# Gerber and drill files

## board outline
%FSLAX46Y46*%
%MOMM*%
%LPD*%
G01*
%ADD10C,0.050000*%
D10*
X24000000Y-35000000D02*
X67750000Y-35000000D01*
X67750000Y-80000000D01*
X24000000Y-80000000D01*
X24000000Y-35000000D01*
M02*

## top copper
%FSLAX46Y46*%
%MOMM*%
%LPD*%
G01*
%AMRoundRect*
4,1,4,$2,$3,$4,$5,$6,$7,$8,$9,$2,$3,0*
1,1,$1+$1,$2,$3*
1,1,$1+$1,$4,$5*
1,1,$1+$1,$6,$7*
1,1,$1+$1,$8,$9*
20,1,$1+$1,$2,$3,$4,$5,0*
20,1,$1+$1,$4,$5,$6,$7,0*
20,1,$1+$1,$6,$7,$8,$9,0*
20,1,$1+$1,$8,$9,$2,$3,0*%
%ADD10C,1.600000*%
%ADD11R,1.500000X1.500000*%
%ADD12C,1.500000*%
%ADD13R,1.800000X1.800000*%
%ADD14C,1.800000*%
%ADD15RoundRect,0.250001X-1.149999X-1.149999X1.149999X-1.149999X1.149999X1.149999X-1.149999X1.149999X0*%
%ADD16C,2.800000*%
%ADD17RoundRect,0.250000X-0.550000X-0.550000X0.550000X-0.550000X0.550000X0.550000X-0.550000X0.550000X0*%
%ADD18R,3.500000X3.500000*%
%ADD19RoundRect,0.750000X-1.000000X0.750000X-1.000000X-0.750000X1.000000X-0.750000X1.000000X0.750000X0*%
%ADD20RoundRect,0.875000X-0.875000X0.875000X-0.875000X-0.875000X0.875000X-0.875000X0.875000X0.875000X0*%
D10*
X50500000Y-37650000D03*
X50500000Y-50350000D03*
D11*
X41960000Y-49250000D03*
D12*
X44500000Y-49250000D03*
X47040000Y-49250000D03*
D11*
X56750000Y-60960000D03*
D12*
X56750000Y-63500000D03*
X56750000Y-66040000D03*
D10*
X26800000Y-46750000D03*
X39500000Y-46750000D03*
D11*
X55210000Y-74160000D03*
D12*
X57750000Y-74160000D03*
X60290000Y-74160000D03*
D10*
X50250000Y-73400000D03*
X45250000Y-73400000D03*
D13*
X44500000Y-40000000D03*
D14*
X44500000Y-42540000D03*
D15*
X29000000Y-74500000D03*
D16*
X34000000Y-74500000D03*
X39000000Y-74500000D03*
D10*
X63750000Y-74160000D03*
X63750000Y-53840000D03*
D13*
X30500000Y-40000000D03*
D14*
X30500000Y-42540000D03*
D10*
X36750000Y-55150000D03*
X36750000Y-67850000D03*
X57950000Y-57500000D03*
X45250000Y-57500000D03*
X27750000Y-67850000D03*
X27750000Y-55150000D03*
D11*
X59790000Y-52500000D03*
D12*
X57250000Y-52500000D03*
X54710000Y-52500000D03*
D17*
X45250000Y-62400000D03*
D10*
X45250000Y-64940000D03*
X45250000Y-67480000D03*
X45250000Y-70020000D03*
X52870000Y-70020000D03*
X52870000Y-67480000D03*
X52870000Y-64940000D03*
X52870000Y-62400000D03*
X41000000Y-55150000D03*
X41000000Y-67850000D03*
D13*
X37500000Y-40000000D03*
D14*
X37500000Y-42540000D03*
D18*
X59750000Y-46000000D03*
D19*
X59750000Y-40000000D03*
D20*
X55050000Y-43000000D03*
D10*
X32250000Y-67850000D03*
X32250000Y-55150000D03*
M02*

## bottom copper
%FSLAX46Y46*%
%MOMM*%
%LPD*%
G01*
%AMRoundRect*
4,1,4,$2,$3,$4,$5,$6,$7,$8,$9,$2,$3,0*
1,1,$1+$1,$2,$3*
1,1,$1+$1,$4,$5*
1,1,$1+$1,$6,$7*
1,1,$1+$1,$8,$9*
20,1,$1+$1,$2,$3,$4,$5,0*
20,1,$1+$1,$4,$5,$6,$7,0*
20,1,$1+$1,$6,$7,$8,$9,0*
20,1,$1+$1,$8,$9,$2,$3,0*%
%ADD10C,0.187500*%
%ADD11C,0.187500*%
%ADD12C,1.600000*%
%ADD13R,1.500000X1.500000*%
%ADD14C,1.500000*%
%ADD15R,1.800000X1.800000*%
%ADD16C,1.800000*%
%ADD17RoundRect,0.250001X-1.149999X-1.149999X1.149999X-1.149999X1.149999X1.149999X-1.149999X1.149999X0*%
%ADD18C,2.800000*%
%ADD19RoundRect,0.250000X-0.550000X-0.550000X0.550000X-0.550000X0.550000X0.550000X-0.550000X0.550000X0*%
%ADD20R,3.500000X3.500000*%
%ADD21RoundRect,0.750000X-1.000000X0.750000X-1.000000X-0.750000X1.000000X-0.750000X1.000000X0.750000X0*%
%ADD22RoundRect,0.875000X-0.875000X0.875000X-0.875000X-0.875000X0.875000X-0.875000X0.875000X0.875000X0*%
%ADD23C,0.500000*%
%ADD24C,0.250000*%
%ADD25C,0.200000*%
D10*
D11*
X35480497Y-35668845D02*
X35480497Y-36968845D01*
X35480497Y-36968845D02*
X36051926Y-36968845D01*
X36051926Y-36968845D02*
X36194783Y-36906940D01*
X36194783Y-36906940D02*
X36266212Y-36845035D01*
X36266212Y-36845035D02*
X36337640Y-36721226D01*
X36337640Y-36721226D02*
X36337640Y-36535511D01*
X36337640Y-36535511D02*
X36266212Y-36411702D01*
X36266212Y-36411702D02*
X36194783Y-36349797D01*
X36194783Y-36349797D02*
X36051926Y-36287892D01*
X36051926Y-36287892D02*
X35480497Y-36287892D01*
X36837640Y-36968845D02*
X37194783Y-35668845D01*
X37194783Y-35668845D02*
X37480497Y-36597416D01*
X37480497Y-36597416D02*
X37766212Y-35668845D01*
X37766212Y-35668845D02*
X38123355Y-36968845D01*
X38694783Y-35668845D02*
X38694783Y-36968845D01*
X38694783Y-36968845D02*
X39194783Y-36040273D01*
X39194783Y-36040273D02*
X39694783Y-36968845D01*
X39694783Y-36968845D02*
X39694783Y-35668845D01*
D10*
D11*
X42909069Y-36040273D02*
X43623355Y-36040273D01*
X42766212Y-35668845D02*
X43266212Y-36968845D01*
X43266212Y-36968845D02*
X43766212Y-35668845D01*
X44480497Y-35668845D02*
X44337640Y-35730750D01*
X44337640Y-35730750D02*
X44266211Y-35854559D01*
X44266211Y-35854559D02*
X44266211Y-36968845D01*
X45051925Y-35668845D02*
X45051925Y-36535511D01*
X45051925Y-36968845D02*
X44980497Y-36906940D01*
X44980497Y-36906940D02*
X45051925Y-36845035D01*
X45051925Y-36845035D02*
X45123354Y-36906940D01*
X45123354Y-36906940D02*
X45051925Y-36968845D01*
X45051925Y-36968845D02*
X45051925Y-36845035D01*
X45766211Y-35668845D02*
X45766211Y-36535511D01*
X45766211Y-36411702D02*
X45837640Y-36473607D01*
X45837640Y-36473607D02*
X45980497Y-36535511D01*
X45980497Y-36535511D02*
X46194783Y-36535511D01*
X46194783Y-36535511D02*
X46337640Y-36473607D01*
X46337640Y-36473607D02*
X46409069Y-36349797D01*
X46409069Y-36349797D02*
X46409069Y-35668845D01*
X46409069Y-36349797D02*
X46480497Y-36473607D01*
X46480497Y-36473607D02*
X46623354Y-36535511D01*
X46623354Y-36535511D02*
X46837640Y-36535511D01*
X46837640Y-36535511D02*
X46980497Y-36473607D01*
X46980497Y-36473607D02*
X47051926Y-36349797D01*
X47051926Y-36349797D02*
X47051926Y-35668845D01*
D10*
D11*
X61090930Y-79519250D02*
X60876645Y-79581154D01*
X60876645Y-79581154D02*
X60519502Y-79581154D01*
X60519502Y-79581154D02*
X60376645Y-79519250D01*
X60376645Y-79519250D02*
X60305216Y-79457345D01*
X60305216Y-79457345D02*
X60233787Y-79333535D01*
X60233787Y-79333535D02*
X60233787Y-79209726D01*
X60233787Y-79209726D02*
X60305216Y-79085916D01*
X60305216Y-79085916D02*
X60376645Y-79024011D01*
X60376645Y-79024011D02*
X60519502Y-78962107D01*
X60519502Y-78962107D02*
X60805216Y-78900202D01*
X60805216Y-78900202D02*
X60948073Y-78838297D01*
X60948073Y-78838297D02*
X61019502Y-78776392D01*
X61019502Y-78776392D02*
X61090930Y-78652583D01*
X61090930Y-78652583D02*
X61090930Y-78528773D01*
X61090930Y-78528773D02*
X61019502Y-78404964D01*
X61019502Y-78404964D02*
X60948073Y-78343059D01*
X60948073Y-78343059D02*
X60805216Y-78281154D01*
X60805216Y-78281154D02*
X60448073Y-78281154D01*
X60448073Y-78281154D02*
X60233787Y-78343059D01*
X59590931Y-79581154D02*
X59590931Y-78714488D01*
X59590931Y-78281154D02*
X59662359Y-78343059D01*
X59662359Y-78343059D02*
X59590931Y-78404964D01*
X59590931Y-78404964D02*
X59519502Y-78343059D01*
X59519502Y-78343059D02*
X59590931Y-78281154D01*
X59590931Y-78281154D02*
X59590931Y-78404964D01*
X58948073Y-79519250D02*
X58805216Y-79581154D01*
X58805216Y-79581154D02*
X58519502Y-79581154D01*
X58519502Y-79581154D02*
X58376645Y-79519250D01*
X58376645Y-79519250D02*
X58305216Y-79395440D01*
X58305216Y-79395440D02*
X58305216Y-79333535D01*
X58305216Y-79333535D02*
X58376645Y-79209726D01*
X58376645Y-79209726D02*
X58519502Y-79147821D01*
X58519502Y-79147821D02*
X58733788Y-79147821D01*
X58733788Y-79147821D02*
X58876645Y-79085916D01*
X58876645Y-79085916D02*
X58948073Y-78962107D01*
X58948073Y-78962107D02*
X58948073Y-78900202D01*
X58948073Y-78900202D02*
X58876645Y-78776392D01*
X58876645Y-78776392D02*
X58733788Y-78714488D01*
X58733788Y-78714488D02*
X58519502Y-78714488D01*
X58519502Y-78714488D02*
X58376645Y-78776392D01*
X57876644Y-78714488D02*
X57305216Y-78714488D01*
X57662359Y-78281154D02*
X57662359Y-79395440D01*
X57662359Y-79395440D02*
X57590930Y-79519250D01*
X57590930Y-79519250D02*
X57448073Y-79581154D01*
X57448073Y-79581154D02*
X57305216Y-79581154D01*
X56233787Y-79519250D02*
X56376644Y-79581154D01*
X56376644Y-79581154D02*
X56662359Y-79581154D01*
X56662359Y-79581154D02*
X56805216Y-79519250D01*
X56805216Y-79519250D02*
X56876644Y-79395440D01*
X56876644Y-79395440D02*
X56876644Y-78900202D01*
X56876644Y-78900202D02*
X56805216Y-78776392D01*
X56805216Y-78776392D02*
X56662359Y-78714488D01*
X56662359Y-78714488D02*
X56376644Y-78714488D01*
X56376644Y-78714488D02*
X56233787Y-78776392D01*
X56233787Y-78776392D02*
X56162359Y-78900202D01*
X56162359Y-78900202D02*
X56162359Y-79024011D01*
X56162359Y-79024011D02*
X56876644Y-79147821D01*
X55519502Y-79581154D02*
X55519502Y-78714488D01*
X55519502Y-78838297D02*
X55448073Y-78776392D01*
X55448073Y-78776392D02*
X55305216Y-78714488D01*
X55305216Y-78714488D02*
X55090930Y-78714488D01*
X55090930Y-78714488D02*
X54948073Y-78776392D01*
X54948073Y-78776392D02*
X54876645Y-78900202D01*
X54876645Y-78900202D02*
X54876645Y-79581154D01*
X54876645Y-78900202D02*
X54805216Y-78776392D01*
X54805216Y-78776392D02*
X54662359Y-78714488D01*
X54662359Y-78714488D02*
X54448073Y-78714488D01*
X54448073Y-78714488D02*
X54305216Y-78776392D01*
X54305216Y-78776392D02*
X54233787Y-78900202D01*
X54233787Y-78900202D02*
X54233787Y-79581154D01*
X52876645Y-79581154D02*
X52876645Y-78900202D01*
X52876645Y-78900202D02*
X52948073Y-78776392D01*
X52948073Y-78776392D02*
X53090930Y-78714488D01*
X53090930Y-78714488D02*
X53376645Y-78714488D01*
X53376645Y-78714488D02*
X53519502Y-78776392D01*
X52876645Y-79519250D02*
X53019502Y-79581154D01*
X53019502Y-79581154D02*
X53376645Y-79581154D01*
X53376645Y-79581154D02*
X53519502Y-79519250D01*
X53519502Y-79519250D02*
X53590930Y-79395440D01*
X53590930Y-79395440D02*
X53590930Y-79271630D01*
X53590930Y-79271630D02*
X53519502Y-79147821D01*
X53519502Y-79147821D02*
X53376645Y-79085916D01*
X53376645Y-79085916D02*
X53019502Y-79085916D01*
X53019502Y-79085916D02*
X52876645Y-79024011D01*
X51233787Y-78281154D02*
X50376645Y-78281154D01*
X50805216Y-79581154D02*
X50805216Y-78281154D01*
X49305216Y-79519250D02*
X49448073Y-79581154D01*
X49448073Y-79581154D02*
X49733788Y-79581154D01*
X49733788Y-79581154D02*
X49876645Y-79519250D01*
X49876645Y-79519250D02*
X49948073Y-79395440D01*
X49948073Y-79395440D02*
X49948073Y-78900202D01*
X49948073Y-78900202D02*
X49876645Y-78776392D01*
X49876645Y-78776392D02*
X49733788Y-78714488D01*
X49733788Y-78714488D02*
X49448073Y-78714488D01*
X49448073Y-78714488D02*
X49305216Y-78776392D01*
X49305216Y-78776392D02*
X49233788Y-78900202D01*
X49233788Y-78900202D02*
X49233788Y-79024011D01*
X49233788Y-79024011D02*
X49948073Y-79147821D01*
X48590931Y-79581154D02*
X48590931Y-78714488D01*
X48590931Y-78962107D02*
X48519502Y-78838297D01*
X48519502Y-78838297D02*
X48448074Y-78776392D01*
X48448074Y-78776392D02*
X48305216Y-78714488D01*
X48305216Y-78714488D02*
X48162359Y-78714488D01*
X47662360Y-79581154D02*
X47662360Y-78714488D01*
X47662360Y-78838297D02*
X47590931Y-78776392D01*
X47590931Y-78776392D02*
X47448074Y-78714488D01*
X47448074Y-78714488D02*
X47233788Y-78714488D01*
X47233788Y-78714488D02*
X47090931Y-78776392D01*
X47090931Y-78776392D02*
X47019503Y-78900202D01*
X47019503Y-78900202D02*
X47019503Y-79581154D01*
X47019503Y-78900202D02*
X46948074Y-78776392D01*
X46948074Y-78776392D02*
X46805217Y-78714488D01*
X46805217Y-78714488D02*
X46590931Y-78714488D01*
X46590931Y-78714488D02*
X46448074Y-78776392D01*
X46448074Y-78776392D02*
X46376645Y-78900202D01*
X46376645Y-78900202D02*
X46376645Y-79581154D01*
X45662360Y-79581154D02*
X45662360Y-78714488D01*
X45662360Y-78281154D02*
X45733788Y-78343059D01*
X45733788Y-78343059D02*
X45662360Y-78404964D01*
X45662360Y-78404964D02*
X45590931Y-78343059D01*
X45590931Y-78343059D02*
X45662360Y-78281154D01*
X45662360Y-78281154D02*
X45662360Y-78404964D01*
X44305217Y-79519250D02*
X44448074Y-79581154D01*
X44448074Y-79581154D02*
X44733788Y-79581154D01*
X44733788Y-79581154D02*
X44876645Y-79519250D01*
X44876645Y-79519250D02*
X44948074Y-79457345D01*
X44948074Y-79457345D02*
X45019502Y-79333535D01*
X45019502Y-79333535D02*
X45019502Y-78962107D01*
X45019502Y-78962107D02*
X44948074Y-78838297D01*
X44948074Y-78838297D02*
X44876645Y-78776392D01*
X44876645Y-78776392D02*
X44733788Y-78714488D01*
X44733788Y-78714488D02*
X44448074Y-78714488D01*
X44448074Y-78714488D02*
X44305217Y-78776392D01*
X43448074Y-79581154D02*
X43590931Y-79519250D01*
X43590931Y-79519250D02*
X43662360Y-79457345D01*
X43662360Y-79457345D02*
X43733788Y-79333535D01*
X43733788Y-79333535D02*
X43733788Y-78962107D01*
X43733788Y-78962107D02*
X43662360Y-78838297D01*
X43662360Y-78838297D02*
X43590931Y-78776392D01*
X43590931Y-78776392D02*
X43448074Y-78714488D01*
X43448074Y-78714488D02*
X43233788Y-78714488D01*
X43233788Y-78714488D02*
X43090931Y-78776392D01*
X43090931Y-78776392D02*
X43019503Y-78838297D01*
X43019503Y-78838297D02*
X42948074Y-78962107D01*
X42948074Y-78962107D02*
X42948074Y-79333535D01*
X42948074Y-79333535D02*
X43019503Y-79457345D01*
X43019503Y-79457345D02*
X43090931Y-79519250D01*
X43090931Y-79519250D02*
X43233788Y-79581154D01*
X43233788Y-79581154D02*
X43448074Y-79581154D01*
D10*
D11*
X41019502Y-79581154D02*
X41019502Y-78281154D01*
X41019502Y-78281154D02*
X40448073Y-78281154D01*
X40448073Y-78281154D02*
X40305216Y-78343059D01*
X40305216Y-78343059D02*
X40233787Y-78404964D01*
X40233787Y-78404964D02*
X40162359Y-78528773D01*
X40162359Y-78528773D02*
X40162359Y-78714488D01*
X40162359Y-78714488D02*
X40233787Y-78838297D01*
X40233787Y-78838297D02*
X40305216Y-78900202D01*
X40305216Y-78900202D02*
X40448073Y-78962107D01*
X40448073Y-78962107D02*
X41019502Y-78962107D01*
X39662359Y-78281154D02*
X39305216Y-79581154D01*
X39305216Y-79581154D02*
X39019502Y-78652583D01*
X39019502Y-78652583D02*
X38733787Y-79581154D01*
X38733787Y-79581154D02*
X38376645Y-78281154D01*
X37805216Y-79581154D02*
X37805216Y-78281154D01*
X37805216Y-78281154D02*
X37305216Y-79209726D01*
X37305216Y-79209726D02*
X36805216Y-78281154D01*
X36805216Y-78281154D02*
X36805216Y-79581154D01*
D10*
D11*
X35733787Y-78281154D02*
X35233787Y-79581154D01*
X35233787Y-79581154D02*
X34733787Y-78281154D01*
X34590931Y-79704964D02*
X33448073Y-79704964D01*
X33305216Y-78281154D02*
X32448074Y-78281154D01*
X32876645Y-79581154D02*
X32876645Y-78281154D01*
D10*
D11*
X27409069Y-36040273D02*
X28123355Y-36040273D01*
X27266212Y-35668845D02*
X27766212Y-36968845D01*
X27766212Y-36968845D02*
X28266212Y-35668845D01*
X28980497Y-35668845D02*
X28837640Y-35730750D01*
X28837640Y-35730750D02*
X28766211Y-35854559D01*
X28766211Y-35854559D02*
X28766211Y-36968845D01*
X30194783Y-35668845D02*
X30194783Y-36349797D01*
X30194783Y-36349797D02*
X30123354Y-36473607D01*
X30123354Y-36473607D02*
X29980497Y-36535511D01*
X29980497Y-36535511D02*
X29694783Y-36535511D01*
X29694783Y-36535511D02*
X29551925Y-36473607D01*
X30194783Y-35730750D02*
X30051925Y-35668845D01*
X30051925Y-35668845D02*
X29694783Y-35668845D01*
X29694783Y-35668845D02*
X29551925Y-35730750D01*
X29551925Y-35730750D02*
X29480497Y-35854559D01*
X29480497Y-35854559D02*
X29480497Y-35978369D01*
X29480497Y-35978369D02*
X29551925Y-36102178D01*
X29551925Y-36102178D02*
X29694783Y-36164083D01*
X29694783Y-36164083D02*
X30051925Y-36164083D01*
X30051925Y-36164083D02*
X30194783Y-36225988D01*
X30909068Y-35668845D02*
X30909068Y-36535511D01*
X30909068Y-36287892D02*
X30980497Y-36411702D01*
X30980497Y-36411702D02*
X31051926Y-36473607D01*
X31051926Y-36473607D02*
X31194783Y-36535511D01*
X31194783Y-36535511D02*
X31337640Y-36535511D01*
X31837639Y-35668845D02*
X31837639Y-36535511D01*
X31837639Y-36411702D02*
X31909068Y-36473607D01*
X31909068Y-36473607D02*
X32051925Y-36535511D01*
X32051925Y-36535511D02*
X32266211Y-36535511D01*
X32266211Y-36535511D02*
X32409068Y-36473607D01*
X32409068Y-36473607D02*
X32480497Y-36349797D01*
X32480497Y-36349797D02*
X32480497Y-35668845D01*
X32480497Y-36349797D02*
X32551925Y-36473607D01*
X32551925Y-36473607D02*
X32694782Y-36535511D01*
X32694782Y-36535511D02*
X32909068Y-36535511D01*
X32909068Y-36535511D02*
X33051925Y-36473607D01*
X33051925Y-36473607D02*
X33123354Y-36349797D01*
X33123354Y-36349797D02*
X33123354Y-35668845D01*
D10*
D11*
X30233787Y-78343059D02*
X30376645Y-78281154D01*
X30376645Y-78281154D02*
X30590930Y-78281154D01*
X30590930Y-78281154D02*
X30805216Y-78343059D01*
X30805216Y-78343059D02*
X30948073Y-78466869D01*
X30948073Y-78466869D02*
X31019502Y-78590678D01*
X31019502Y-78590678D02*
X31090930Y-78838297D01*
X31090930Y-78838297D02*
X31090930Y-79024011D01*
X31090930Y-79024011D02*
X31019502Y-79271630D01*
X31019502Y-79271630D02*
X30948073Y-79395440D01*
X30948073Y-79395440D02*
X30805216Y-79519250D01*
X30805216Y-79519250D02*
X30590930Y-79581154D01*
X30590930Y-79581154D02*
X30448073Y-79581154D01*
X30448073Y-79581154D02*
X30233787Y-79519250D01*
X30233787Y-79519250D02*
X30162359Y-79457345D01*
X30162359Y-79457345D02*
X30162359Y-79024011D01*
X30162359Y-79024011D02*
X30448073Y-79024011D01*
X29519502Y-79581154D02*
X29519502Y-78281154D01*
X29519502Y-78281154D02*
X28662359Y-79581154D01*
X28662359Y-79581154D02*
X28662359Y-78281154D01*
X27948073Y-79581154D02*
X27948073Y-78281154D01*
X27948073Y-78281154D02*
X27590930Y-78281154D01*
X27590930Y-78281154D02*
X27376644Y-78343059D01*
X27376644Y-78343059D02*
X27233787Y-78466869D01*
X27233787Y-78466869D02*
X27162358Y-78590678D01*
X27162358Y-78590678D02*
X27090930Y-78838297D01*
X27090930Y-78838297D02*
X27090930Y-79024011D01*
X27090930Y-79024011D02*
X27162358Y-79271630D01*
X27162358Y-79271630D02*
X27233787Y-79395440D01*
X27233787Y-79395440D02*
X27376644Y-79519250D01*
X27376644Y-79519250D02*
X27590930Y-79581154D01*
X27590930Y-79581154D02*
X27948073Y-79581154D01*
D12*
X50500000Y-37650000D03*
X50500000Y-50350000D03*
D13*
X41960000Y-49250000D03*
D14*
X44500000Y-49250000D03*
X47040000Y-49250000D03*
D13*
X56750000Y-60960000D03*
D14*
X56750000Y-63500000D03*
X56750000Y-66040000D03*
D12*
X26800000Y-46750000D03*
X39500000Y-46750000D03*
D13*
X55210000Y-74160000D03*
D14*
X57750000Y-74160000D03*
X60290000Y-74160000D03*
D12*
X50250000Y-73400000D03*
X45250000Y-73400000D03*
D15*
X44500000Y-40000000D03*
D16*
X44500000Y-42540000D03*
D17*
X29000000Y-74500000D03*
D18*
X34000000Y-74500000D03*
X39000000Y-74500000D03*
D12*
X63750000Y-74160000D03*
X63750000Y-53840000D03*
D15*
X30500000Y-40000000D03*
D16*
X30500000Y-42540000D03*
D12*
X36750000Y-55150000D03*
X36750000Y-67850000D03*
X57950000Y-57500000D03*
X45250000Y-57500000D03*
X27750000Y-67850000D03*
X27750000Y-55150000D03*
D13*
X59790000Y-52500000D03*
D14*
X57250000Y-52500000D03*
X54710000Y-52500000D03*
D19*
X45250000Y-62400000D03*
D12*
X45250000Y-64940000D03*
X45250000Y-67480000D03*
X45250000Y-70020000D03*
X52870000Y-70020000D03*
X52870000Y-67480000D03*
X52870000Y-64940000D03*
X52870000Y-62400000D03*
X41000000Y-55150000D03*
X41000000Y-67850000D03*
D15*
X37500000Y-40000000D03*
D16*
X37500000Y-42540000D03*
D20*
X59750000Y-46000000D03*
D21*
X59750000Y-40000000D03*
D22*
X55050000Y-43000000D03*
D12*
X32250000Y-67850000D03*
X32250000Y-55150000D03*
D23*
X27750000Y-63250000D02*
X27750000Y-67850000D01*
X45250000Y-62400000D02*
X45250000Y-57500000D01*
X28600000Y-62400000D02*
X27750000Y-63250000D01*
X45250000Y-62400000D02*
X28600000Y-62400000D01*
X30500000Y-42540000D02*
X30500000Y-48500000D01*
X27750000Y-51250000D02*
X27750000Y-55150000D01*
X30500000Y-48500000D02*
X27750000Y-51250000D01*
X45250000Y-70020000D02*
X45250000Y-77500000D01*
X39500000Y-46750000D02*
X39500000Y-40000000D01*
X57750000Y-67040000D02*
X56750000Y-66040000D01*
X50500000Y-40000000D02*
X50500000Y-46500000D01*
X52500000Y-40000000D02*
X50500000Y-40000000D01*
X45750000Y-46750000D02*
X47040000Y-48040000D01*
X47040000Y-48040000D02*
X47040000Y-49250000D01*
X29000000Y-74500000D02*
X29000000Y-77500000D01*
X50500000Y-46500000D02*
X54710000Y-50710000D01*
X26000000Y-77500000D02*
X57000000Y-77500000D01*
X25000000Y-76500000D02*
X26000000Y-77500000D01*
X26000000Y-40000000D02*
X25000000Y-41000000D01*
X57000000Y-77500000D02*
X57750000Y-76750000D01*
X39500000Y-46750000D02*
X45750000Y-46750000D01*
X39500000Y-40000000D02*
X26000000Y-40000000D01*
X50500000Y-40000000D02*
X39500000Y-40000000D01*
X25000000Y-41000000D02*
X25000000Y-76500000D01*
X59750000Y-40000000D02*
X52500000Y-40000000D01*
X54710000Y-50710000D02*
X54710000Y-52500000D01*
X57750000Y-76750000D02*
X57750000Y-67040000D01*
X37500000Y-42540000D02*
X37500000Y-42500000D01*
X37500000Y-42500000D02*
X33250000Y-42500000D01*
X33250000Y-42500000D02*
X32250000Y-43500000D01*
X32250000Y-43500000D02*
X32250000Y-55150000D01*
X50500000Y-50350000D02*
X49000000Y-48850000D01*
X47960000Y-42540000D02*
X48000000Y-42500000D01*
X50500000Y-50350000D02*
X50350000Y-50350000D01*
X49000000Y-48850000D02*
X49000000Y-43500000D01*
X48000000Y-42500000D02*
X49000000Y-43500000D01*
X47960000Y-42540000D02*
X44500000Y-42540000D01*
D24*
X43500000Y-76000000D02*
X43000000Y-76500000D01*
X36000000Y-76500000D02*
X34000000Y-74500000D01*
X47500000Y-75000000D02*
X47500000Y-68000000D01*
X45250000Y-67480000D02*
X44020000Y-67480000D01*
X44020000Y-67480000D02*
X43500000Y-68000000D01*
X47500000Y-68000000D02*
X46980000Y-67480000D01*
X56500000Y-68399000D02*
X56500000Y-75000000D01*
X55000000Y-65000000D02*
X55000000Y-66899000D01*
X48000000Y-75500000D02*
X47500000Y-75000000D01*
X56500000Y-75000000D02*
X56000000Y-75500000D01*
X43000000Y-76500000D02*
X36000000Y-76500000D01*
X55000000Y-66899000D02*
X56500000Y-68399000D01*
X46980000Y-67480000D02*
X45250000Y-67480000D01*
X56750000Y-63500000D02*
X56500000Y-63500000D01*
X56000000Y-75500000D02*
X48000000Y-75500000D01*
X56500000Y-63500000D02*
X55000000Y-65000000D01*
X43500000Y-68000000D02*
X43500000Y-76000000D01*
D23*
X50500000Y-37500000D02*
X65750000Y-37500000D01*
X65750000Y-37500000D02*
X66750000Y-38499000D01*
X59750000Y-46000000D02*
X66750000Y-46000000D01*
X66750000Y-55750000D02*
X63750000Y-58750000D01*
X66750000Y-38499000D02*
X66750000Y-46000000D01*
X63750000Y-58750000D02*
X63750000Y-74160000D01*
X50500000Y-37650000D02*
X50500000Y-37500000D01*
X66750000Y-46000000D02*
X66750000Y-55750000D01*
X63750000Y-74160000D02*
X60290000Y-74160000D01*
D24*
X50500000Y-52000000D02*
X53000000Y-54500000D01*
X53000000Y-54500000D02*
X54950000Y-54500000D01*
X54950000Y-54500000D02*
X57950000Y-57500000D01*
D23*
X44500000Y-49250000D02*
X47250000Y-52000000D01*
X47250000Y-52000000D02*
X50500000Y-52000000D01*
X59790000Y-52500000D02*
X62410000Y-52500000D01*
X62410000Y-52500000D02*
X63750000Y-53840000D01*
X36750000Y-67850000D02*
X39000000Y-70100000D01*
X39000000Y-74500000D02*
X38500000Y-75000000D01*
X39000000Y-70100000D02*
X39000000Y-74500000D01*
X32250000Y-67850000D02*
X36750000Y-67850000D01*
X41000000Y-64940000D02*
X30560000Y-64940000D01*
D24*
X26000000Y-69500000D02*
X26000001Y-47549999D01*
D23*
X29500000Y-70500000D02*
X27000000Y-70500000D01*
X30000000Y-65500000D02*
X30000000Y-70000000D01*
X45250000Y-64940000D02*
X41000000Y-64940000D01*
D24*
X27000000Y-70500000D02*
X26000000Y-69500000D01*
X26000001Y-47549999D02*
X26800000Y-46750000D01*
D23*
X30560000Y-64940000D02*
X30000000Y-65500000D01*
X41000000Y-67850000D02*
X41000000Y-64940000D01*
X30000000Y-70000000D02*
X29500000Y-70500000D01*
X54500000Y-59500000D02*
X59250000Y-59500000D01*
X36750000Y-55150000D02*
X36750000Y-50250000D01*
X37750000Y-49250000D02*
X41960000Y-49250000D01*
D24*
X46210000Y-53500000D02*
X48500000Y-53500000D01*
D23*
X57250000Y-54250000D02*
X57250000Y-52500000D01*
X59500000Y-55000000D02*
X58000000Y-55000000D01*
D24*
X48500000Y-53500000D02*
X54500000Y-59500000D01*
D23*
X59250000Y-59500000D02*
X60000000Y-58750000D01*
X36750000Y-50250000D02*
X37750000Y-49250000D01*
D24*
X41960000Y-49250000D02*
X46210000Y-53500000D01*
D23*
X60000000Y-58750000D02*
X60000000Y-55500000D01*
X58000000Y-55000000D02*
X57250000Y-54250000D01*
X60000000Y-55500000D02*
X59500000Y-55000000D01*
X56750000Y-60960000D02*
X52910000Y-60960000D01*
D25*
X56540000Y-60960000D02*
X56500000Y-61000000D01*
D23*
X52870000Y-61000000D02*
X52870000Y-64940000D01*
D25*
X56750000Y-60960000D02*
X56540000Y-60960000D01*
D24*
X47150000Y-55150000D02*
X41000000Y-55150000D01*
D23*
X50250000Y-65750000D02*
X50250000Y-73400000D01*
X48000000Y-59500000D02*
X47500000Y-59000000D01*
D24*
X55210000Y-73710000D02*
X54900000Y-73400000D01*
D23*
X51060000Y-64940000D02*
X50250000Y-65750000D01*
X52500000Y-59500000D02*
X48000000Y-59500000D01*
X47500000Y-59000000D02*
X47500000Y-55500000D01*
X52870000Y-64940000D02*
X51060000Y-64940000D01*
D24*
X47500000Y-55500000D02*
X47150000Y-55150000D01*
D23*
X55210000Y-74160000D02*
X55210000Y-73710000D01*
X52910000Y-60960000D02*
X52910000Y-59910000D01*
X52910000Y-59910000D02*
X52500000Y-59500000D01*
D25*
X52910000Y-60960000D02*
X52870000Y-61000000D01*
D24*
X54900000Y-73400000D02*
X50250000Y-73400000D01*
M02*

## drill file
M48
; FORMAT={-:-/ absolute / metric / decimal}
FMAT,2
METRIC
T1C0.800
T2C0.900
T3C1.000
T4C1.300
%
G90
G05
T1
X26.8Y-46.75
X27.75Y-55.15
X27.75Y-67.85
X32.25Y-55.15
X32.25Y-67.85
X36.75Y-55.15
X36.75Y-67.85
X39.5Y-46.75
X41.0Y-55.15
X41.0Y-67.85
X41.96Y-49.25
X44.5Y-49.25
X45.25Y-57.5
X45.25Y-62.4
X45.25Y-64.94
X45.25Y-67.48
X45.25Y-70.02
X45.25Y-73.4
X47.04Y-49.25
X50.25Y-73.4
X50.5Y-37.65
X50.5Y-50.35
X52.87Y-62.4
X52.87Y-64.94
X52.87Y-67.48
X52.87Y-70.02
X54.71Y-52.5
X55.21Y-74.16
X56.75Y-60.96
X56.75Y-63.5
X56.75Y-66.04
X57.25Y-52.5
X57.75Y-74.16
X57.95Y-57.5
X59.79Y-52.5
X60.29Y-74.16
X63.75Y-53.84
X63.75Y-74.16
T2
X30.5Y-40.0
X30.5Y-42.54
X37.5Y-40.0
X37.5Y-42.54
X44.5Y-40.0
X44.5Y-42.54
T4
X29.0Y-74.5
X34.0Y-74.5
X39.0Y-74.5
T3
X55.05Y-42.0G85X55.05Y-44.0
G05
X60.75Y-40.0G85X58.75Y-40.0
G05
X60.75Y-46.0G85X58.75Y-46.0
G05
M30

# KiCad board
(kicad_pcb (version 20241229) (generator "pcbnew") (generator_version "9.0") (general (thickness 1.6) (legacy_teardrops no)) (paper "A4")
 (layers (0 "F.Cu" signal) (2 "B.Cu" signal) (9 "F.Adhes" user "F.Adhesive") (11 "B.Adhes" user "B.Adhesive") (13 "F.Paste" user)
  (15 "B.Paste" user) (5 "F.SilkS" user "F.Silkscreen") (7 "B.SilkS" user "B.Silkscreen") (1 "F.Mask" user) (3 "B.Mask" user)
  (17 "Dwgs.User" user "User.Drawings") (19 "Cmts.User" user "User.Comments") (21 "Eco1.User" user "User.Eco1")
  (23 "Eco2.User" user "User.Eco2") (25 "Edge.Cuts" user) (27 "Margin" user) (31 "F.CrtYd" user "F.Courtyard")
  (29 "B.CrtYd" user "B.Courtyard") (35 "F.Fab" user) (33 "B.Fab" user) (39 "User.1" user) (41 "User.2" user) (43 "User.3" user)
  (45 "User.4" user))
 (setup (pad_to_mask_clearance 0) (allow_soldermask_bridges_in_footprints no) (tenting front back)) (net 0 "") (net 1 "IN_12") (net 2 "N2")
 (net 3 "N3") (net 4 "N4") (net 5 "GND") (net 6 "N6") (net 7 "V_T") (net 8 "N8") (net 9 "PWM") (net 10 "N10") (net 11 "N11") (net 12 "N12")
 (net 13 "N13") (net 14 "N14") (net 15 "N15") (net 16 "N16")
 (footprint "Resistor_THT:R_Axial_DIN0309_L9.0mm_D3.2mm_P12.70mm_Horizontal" (layer "F.Cu") (at 50.5 37.65 -90)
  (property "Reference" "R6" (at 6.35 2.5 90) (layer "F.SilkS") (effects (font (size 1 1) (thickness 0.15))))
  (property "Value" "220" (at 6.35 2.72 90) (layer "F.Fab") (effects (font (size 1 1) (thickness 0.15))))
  (pad "1" thru_hole circle (at 0 0 270) (size 1.6 1.6) (drill 0.8) (layers "*.Cu" "*.Mask") (remove_unused_layers no) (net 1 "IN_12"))
  (pad "2" thru_hole circle (at 12.7 0 270) (size 1.6 1.6) (drill 0.8) (layers "*.Cu" "*.Mask") (remove_unused_layers no) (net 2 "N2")))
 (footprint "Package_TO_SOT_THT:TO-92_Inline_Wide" (layer "F.Cu") (at 41.96 49.25)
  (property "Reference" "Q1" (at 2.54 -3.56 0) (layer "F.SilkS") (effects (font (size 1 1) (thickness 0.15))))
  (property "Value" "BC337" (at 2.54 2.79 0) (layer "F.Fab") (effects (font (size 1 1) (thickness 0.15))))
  (pad "1" thru_hole rect (at 0 0) (size 1.5 1.5) (drill 0.8) (layers "*.Cu" "*.Mask") (remove_unused_layers no) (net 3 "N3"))
  (pad "2" thru_hole circle (at 2.54 0) (size 1.5 1.5) (drill 0.8) (layers "*.Cu" "*.Mask") (remove_unused_layers no) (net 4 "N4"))
  (pad "3" thru_hole circle (at 5.08 0) (size 1.5 1.5) (drill 0.8) (layers "*.Cu" "*.Mask") (remove_unused_layers no) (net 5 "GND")))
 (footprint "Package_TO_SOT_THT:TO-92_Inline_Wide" (layer "F.Cu") (at 56.75 60.96 -90)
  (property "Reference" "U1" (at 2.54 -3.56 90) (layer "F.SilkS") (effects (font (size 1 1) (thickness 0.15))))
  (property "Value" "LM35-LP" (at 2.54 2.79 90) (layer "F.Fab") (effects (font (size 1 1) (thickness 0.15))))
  (pad "1" thru_hole rect (at 0 0 270) (size 1.5 1.5) (drill 0.8) (layers "*.Cu" "*.Mask") (remove_unused_layers no) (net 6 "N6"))
  (pad "2" thru_hole circle (at 2.54 0 270) (size 1.5 1.5) (drill 0.8) (layers "*.Cu" "*.Mask") (remove_unused_layers no) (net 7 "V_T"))
  (pad "3" thru_hole circle (at 5.08 0 270) (size 1.5 1.5) (drill 0.8) (layers "*.Cu" "*.Mask") (remove_unused_layers no) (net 5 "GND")))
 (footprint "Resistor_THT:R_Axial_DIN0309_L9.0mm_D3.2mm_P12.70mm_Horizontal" (layer "F.Cu") (at 26.8 46.75)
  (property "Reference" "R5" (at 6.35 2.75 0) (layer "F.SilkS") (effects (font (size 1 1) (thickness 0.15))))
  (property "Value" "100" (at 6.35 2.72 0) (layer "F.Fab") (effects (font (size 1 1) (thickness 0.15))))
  (pad "1" thru_hole circle (at 0 0) (size 1.6 1.6) (drill 0.8) (layers "*.Cu" "*.Mask") (remove_unused_layers no) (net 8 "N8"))
  (pad "2" thru_hole circle (at 12.7 0) (size 1.6 1.6) (drill 0.8) (layers "*.Cu" "*.Mask") (remove_unused_layers no) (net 5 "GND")))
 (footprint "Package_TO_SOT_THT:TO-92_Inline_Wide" (layer "F.Cu") (at 55.21 74.16)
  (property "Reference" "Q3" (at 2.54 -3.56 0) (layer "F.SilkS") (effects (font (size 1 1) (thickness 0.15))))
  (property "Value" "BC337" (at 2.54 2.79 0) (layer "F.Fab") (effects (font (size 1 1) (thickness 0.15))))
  (pad "1" thru_hole rect (at 0 0) (size 1.5 1.5) (drill 0.8) (layers "*.Cu" "*.Mask") (remove_unused_layers no) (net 6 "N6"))
  (pad "2" thru_hole circle (at 2.54 0) (size 1.5 1.5) (drill 0.8) (layers "*.Cu" "*.Mask") (remove_unused_layers no) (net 5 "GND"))
  (pad "3" thru_hole circle (at 5.08 0) (size 1.5 1.5) (drill 0.8) (layers "*.Cu" "*.Mask") (remove_unused_layers no) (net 1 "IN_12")))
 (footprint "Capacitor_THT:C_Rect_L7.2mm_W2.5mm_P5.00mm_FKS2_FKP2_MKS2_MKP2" (layer "F.Cu") (at 50.25 73.4 180)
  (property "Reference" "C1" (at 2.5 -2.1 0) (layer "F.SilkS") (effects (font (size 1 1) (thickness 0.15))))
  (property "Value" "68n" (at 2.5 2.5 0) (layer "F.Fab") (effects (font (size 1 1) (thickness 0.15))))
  (pad "1" thru_hole circle (at 0 0 180) (size 1.6 1.6) (drill 0.8) (layers "*.Cu" "*.Mask") (remove_unused_layers no) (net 6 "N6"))
  (pad "2" thru_hole circle (at 5 0 180) (size 1.6 1.6) (drill 0.8) (layers "*.Cu" "*.Mask") (remove_unused_layers no) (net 5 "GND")))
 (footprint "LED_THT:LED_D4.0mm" (layer "F.Cu") (at 44.5 40 -90)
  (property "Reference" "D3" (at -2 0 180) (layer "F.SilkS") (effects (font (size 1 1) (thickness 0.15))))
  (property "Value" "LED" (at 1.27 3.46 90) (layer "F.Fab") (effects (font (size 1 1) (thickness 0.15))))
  (pad "1" thru_hole rect (at 0 0 270) (size 1.8 1.8) (drill 0.9) (layers "*.Cu" "*.Mask") (remove_unused_layers no) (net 5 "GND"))
  (pad "2" thru_hole circle (at 2.54 0 270) (size 1.8 1.8) (drill 0.9) (layers "*.Cu" "*.Mask") (remove_unused_layers no) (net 2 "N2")))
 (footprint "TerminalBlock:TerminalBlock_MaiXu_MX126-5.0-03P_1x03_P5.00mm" (layer "F.Cu") (at 29 74.5)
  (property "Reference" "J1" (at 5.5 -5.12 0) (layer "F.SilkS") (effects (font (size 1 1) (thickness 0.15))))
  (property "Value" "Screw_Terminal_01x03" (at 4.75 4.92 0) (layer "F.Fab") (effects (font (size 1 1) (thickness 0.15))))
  (pad "1" thru_hole roundrect (at 0 0) (size 2.8 2.8) (drill 1.3) (layers "*.Cu" "*.Mask") (remove_unused_layers no)
   (roundrect_rratio 0.089286) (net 5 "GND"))
  (pad "2" thru_hole circle (at 5 0) (size 2.8 2.8) (drill 1.3) (layers "*.Cu" "*.Mask") (remove_unused_layers no) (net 7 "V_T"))
  (pad "3" thru_hole circle (at 10 0) (size 2.8 2.8) (drill 1.3) (layers "*.Cu" "*.Mask") (remove_unused_layers no) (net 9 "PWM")))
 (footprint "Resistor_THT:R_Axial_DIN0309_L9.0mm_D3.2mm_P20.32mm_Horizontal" (layer "F.Cu") (at 63.75 74.16 90)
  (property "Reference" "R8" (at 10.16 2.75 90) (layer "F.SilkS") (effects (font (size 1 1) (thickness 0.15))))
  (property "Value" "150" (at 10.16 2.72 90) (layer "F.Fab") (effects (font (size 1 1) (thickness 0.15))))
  (pad "1" thru_hole circle (at 0 0 90) (size 1.6 1.6) (drill 0.8) (layers "*.Cu" "*.Mask") (remove_unused_layers no) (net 1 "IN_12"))
  (pad "2" thru_hole circle (at 20.32 0 90) (size 1.6 1.6) (drill 0.8) (layers "*.Cu" "*.Mask") (remove_unused_layers no) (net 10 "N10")))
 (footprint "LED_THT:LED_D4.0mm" (layer "F.Cu") (at 30.5 40 -90)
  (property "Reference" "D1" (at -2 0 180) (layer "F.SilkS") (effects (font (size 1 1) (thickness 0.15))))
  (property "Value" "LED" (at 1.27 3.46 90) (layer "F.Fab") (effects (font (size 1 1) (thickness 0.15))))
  (pad "1" thru_hole rect (at 0 0 270) (size 1.8 1.8) (drill 0.9) (layers "*.Cu" "*.Mask") (remove_unused_layers no) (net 5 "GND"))
  (pad "2" thru_hole circle (at 2.54 0 270) (size 1.8 1.8) (drill 0.9) (layers "*.Cu" "*.Mask") (remove_unused_layers no) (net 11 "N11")))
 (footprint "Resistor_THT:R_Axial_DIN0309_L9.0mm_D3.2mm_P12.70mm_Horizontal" (layer "F.Cu") (at 36.75 55.15 -90)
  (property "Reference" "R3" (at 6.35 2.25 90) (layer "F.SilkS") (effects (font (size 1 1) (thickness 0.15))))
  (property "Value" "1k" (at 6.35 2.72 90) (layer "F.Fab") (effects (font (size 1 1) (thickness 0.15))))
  (pad "1" thru_hole circle (at 0 0 270) (size 1.6 1.6) (drill 0.8) (layers "*.Cu" "*.Mask") (remove_unused_layers no) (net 3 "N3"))
  (pad "2" thru_hole circle (at 12.7 0 270) (size 1.6 1.6) (drill 0.8) (layers "*.Cu" "*.Mask") (remove_unused_layers no) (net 9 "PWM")))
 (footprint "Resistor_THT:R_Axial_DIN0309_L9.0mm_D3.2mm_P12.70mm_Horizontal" (layer "F.Cu") (at 57.95 57.5 180)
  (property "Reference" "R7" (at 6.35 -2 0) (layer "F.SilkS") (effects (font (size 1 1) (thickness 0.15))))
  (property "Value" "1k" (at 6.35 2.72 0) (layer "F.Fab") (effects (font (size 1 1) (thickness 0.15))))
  (pad "1" thru_hole circle (at 0 0 180) (size 1.6 1.6) (drill 0.8) (layers "*.Cu" "*.Mask") (remove_unused_layers no) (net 4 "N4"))
  (pad "2" thru_hole circle (at 12.7 0 180) (size 1.6 1.6) (drill 0.8) (layers "*.Cu" "*.Mask") (remove_unused_layers no) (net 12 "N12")))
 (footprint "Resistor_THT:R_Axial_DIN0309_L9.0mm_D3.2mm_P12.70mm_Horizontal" (layer "F.Cu") (at 27.75 67.85 90)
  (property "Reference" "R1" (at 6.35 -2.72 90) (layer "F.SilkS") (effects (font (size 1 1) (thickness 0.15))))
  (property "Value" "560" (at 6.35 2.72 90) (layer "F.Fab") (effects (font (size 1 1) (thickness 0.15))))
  (pad "1" thru_hole circle (at 0 0 90) (size 1.6 1.6) (drill 0.8) (layers "*.Cu" "*.Mask") (remove_unused_layers no) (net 12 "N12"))
  (pad "2" thru_hole circle (at 12.7 0 90) (size 1.6 1.6) (drill 0.8) (layers "*.Cu" "*.Mask") (remove_unused_layers no) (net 11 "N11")))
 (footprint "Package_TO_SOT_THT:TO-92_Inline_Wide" (layer "F.Cu") (at 59.79 52.5 180)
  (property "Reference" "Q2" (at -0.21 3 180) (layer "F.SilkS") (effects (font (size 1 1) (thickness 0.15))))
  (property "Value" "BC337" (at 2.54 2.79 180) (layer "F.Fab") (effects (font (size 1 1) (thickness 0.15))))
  (pad "1" thru_hole rect (at 0 0 180) (size 1.5 1.5) (drill 0.8) (layers "*.Cu" "*.Mask") (remove_unused_layers no) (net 10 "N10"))
  (pad "2" thru_hole circle (at 2.54 0 180) (size 1.5 1.5) (drill 0.8) (layers "*.Cu" "*.Mask") (remove_unused_layers no) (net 3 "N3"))
  (pad "3" thru_hole circle (at 5.08 0 180) (size 1.5 1.5) (drill 0.8) (layers "*.Cu" "*.Mask") (remove_unused_layers no) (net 5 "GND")))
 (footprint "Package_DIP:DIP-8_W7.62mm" (layer "F.Cu") (at 45.25 62.4)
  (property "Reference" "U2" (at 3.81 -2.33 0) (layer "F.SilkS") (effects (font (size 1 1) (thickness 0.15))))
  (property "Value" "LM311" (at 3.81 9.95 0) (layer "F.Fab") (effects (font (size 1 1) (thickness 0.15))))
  (pad "1" thru_hole roundrect (at 0 0) (size 1.6 1.6) (drill 0.8) (layers "*.Cu" "*.Mask") (remove_unused_layers no)
   (roundrect_rratio 0.15625) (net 12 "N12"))
  (pad "2" thru_hole circle (at 0 2.54) (size 1.6 1.6) (drill 0.8) (layers "*.Cu" "*.Mask") (remove_unused_layers no) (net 8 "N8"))
  (pad "3" thru_hole circle (at 0 5.08) (size 1.6 1.6) (drill 0.8) (layers "*.Cu" "*.Mask") (remove_unused_layers no) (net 7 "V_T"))
  (pad "4" thru_hole circle (at 0 7.62) (size 1.6 1.6) (drill 0.8) (layers "*.Cu" "*.Mask") (remove_unused_layers no) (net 5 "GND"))
  (pad "5" thru_hole circle (at 7.62 7.62) (size 1.6 1.6) (drill 0.8) (layers "*.Cu" "*.Mask") (remove_unused_layers no) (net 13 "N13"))
  (pad "6" thru_hole circle (at 7.62 5.08) (size 1.6 1.6) (drill 0.8) (layers "*.Cu" "*.Mask") (remove_unused_layers no) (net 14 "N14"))
  (pad "7" thru_hole circle (at 7.62 2.54) (size 1.6 1.6) (drill 0.8) (layers "*.Cu" "*.Mask") (remove_unused_layers no) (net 6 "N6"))
  (pad "8" thru_hole circle (at 7.62 0) (size 1.6 1.6) (drill 0.8) (layers "*.Cu" "*.Mask") (remove_unused_layers no) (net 6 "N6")))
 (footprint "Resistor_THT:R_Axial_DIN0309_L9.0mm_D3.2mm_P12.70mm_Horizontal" (layer "F.Cu") (at 41 55.15 -90)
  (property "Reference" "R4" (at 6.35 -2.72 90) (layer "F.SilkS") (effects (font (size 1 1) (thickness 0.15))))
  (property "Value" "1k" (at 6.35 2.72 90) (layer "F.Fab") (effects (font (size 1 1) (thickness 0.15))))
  (pad "1" thru_hole circle (at 0 0 270) (size 1.6 1.6) (drill 0.8) (layers "*.Cu" "*.Mask") (remove_unused_layers no) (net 6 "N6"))
  (pad "2" thru_hole circle (at 12.7 0 270) (size 1.6 1.6) (drill 0.8) (layers "*.Cu" "*.Mask") (remove_unused_layers no) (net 8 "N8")))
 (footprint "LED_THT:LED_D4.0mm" (layer "F.Cu") (at 37.5 40 -90)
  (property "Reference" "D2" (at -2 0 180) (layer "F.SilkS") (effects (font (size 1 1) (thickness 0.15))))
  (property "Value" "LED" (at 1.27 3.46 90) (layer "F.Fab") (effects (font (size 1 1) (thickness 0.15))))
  (pad "1" thru_hole rect (at 0 0 270) (size 1.8 1.8) (drill 0.9) (layers "*.Cu" "*.Mask") (remove_unused_layers no) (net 5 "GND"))
  (pad "2" thru_hole circle (at 2.54 0 270) (size 1.8 1.8) (drill 0.9) (layers "*.Cu" "*.Mask") (remove_unused_layers no) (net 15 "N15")))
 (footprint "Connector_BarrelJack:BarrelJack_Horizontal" (layer "F.Cu") (at 59.75 46 -90)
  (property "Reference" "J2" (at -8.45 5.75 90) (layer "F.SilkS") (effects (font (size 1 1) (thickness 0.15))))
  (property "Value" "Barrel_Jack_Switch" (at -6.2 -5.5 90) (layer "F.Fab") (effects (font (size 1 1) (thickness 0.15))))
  (pad "1" thru_hole rect (at 0 0 270) (size 3.5 3.5) (drill oval 1 3) (layers "*.Cu" "*.Mask") (remove_unused_layers no) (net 1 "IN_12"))
  (pad "2" thru_hole roundrect (at -6 0 270) (size 3 3.5) (drill oval 1 3) (layers "*.Cu" "*.Mask") (remove_unused_layers no)
   (roundrect_rratio 0.25) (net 5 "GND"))
  (pad "3" thru_hole roundrect (at -3 4.7 270) (size 3.5 3.5) (drill oval 3 1) (layers "*.Cu" "*.Mask") (remove_unused_layers no)
   (roundrect_rratio 0.25) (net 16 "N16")))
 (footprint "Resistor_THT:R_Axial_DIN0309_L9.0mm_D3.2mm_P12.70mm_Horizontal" (layer "F.Cu") (at 32.25 67.85 90)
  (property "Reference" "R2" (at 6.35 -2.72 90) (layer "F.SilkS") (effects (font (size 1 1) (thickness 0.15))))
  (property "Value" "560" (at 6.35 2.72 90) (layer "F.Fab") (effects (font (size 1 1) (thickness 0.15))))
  (pad "1" thru_hole circle (at 0 0 90) (size 1.6 1.6) (drill 0.8) (layers "*.Cu" "*.Mask") (remove_unused_layers no) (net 9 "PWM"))
  (pad "2" thru_hole circle (at 12.7 0 90) (size 1.6 1.6) (drill 0.8) (layers "*.Cu" "*.Mask") (remove_unused_layers no) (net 15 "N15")))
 (gr_rect (start 24 35) (end 67.75 80) (stroke (width 0.05) (type solid)) (fill no) (layer "Edge.Cuts"))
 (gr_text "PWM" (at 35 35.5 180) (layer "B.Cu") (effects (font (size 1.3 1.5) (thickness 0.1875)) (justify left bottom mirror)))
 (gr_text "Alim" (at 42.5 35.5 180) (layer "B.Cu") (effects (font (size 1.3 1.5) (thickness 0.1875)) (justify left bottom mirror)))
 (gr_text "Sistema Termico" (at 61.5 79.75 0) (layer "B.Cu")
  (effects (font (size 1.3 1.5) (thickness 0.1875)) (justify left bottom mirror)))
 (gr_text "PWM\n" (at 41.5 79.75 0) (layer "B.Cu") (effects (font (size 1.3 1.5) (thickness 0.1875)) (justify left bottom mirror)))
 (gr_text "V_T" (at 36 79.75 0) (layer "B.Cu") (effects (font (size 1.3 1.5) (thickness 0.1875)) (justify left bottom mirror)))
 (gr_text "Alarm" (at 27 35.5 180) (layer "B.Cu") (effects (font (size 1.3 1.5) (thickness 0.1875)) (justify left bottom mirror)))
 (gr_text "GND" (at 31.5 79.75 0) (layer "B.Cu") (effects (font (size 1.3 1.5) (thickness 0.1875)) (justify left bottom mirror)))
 (segment (start 27.75 63.25) (end 27.75 67.85) (width 0.5) (layer "B.Cu") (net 12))
 (segment (start 45.25 62.4) (end 45.25 57.5) (width 0.5) (layer "B.Cu") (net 12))
 (segment (start 28.6 62.4) (end 27.75 63.25) (width 0.5) (layer "B.Cu") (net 12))
 (segment (start 45.25 62.4) (end 28.6 62.4) (width 0.5) (layer "B.Cu") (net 12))
 (segment (start 30.5 42.54) (end 30.5 48.5) (width 0.5) (layer "B.Cu") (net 11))
 (segment (start 27.75 51.25) (end 27.75 55.15) (width 0.5) (layer "B.Cu") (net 11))
 (segment (start 30.5 48.5) (end 27.75 51.25) (width 0.5) (layer "B.Cu") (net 11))
 (segment (start 45.25 70.02) (end 45.25 77.5) (width 0.5) (layer "B.Cu") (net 5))
 (segment (start 39.5 46.75) (end 39.5 40) (width 0.5) (layer "B.Cu") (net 5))
 (segment (start 57.75 67.04) (end 56.75 66.04) (width 0.5) (layer "B.Cu") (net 5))
 (segment (start 50.5 40) (end 50.5 46.5) (width 0.5) (layer "B.Cu") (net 5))
 (segment (start 52.5 40) (end 50.5 40) (width 0.5) (layer "B.Cu") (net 5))
 (segment (start 45.75 46.75) (end 47.04 48.04) (width 0.5) (layer "B.Cu") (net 5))
 (segment (start 47.04 48.04) (end 47.04 49.25) (width 0.5) (layer "B.Cu") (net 5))
 (segment (start 29 74.5) (end 29 77.5) (width 0.5) (layer "B.Cu") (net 5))
 (segment (start 50.5 46.5) (end 54.71 50.71) (width 0.5) (layer "B.Cu") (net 5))
 (segment (start 26 77.5) (end 57 77.5) (width 0.5) (layer "B.Cu") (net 5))
 (segment (start 25 76.5) (end 26 77.5) (width 0.5) (layer "B.Cu") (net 5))
 (segment (start 26 40) (end 25 41) (width 0.5) (layer "B.Cu") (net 5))
 (segment (start 57 77.5) (end 57.75 76.75) (width 0.5) (layer "B.Cu") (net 5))
 (segment (start 39.5 46.75) (end 45.75 46.75) (width 0.5) (layer "B.Cu") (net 5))
 (segment (start 39.5 40) (end 26 40) (width 0.5) (layer "B.Cu") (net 5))
 (segment (start 50.5 40) (end 39.5 40) (width 0.5) (layer "B.Cu") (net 5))
 (segment (start 25 41) (end 25 76.5) (width 0.5) (layer "B.Cu") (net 5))
 (segment (start 59.75 40) (end 52.5 40) (width 0.5) (layer "B.Cu") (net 5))
 (segment (start 54.71 50.71) (end 54.71 52.5) (width 0.5) (layer "B.Cu") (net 5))
 (segment (start 57.75 76.75) (end 57.75 67.04) (width 0.5) (layer "B.Cu") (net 5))
 (segment (start 37.5 42.54) (end 37.5 42.5) (width 0.5) (layer "B.Cu") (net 15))
 (segment (start 37.5 42.5) (end 33.25 42.5) (width 0.5) (layer "B.Cu") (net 15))
 (segment (start 33.25 42.5) (end 32.25 43.5) (width 0.5) (layer "B.Cu") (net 15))
 (segment (start 32.25 43.5) (end 32.25 55.15) (width 0.5) (layer "B.Cu") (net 15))
 (segment (start 50.5 50.35) (end 49 48.85) (width 0.5) (layer "B.Cu") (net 2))
 (segment (start 47.96 42.54) (end 48 42.5) (width 0.5) (layer "B.Cu") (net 2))
 (segment (start 50.5 50.35) (end 50.35 50.35) (width 0.5) (layer "B.Cu") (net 2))
 (segment (start 49 48.85) (end 49 43.5) (width 0.5) (layer "B.Cu") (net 2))
 (segment (start 48 42.5) (end 49 43.5) (width 0.5) (layer "B.Cu") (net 2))
 (segment (start 47.96 42.54) (end 44.5 42.54) (width 0.5) (layer "B.Cu") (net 2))
 (segment (start 43.5 76) (end 43 76.5) (width 0.25) (layer "B.Cu") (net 7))
 (segment (start 36 76.5) (end 34 74.5) (width 0.25) (layer "B.Cu") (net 7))
 (segment (start 47.5 75) (end 47.5 68) (width 0.25) (layer "B.Cu") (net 7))
 (segment (start 45.25 67.48) (end 44.02 67.48) (width 0.25) (layer "B.Cu") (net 7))
 (segment (start 44.02 67.48) (end 43.5 68) (width 0.25) (layer "B.Cu") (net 7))
 (segment (start 47.5 68) (end 46.98 67.48) (width 0.25) (layer "B.Cu") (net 7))
 (segment (start 56.5 68.399) (end 56.5 75) (width 0.25) (layer "B.Cu") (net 7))
 (segment (start 55 65) (end 55 66.899) (width 0.25) (layer "B.Cu") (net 7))
 (segment (start 48 75.5) (end 47.5 75) (width 0.25) (layer "B.Cu") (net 7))
 (segment (start 56.5 75) (end 56 75.5) (width 0.25) (layer "B.Cu") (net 7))
 (segment (start 43 76.5) (end 36 76.5) (width 0.25) (layer "B.Cu") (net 7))
 (segment (start 55 66.899) (end 56.5 68.399) (width 0.25) (layer "B.Cu") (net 7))
 (segment (start 46.98 67.48) (end 45.25 67.48) (width 0.25) (layer "B.Cu") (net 7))
 (segment (start 56.75 63.5) (end 56.5 63.5) (width 0.25) (layer "B.Cu") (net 7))
 (segment (start 56 75.5) (end 48 75.5) (width 0.25) (layer "B.Cu") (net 7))
 (segment (start 56.5 63.5) (end 55 65) (width 0.25) (layer "B.Cu") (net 7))
 (segment (start 43.5 68) (end 43.5 76) (width 0.25) (layer "B.Cu") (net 7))
 (segment (start 50.5 37.5) (end 65.75 37.5) (width 0.5) (layer "B.Cu") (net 1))
 (segment (start 65.75 37.5) (end 66.75 38.499) (width 0.5) (layer "B.Cu") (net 1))
 (segment (start 59.75 46) (end 66.75 46) (width 0.5) (layer "B.Cu") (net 1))
 (segment (start 66.75 55.75) (end 63.75 58.75) (width 0.5) (layer "B.Cu") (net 1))
 (segment (start 66.75 38.499) (end 66.75 46) (width 0.5) (layer "B.Cu") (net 1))
 (segment (start 63.75 58.75) (end 63.75 74.16) (width 0.5) (layer "B.Cu") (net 1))
 (segment (start 50.5 37.65) (end 50.5 37.5) (width 0.5) (layer "B.Cu") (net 1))
 (segment (start 66.75 46) (end 66.75 55.75) (width 0.5) (layer "B.Cu") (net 1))
 (segment (start 63.75 74.16) (end 60.29 74.16) (width 0.5) (layer "B.Cu") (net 1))
 (segment (start 50.5 52) (end 53 54.5) (width 0.25) (layer "B.Cu") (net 4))
 (segment (start 53 54.5) (end 54.95 54.5) (width 0.25) (layer "B.Cu") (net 4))
 (segment (start 54.95 54.5) (end 57.95 57.5) (width 0.25) (layer "B.Cu") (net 4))
 (segment (start 44.5 49.25) (end 47.25 52) (width 0.5) (layer "B.Cu") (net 4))
 (segment (start 47.25 52) (end 50.5 52) (width 0.5) (layer "B.Cu") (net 4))
 (segment (start 59.79 52.5) (end 62.41 52.5) (width 0.5) (layer "B.Cu") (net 10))
 (segment (start 62.41 52.5) (end 63.75 53.84) (width 0.5) (layer "B.Cu") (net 10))
 (segment (start 36.75 67.85) (end 39 70.1) (width 0.5) (layer "B.Cu") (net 9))
 (segment (start 39 74.5) (end 38.5 75) (width 0.5) (layer "B.Cu") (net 9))
 (segment (start 39 70.1) (end 39 74.5) (width 0.5) (layer "B.Cu") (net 9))
 (segment (start 32.25 67.85) (end 36.75 67.85) (width 0.5) (layer "B.Cu") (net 9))
 (segment (start 41 64.94) (end 30.56 64.94) (width 0.5) (layer "B.Cu") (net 8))
 (segment (start 26 69.5) (end 26.000001 47.549999) (width 0.25) (layer "B.Cu") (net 8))
 (segment (start 29.5 70.5) (end 27 70.5) (width 0.5) (layer "B.Cu") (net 8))
 (segment (start 30 65.5) (end 30 70) (width 0.5) (layer "B.Cu") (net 8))
 (segment (start 45.25 64.94) (end 41 64.94) (width 0.5) (layer "B.Cu") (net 8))
 (segment (start 27 70.5) (end 26 69.5) (width 0.25) (layer "B.Cu") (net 8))
 (segment (start 26.000001 47.549999) (end 26.8 46.75) (width 0.25) (layer "B.Cu") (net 8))
 (segment (start 30.56 64.94) (end 30 65.5) (width 0.5) (layer "B.Cu") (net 8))
 (segment (start 41 67.85) (end 41 64.94) (width 0.5) (layer "B.Cu") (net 8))
 (segment (start 30 70) (end 29.5 70.5) (width 0.5) (layer "B.Cu") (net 8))
 (segment (start 54.5 59.5) (end 59.25 59.5) (width 0.5) (layer "B.Cu") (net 3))
 (segment (start 36.75 55.15) (end 36.75 50.25) (width 0.5) (layer "B.Cu") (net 3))
 (segment (start 37.75 49.25) (end 41.96 49.25) (width 0.5) (layer "B.Cu") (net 3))
 (segment (start 46.21 53.5) (end 48.5 53.5) (width 0.25) (layer "B.Cu") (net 3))
 (segment (start 57.25 54.25) (end 57.25 52.5) (width 0.5) (layer "B.Cu") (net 3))
 (segment (start 59.5 55) (end 58 55) (width 0.5) (layer "B.Cu") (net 3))
 (segment (start 48.5 53.5) (end 54.5 59.5) (width 0.25) (layer "B.Cu") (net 3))
 (segment (start 59.25 59.5) (end 60 58.75) (width 0.5) (layer "B.Cu") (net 3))
 (segment (start 36.75 50.25) (end 37.75 49.25) (width 0.5) (layer "B.Cu") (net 3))
 (segment (start 41.96 49.25) (end 46.21 53.5) (width 0.25) (layer "B.Cu") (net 3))
 (segment (start 60 58.75) (end 60 55.5) (width 0.5) (layer "B.Cu") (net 3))
 (segment (start 58 55) (end 57.25 54.25) (width 0.5) (layer "B.Cu") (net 3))
 (segment (start 60 55.5) (end 59.5 55) (width 0.5) (layer "B.Cu") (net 3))
 (segment (start 56.75 60.96) (end 52.91 60.96) (width 0.5) (layer "B.Cu") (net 6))
 (segment (start 56.54 60.96) (end 56.5 61) (width 0.2) (layer "B.Cu") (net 6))
 (segment (start 52.87 61) (end 52.87 64.94) (width 0.5) (layer "B.Cu") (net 6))
 (segment (start 56.75 60.96) (end 56.54 60.96) (width 0.2) (layer "B.Cu") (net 6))
 (segment (start 47.15 55.15) (end 41 55.15) (width 0.25) (layer "B.Cu") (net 6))
 (segment (start 50.25 65.75) (end 50.25 73.4) (width 0.5) (layer "B.Cu") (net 6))
 (segment (start 48 59.5) (end 47.5 59) (width 0.5) (layer "B.Cu") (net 6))
 (segment (start 55.21 73.71) (end 54.9 73.4) (width 0.25) (layer "B.Cu") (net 6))
 (segment (start 51.06 64.94) (end 50.25 65.75) (width 0.5) (layer "B.Cu") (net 6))
 (segment (start 52.5 59.5) (end 48 59.5) (width 0.5) (layer "B.Cu") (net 6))
 (segment (start 47.5 59) (end 47.5 55.5) (width 0.5) (layer "B.Cu") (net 6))
 (segment (start 52.87 64.94) (end 51.06 64.94) (width 0.5) (layer "B.Cu") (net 6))
 (segment (start 47.5 55.5) (end 47.15 55.15) (width 0.25) (layer "B.Cu") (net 6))
 (segment (start 55.21 74.16) (end 55.21 73.71) (width 0.5) (layer "B.Cu") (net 6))
 (segment (start 52.91 60.96) (end 52.91 59.91) (width 0.5) (layer "B.Cu") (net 6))
 (segment (start 52.91 59.91) (end 52.5 59.5) (width 0.5) (layer "B.Cu") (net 6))
 (segment (start 52.91 60.96) (end 52.87 61) (width 0.2) (layer "B.Cu") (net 6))
 (segment (start 54.9 73.4) (end 50.25 73.4) (width 0.25) (layer "B.Cu") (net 6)))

